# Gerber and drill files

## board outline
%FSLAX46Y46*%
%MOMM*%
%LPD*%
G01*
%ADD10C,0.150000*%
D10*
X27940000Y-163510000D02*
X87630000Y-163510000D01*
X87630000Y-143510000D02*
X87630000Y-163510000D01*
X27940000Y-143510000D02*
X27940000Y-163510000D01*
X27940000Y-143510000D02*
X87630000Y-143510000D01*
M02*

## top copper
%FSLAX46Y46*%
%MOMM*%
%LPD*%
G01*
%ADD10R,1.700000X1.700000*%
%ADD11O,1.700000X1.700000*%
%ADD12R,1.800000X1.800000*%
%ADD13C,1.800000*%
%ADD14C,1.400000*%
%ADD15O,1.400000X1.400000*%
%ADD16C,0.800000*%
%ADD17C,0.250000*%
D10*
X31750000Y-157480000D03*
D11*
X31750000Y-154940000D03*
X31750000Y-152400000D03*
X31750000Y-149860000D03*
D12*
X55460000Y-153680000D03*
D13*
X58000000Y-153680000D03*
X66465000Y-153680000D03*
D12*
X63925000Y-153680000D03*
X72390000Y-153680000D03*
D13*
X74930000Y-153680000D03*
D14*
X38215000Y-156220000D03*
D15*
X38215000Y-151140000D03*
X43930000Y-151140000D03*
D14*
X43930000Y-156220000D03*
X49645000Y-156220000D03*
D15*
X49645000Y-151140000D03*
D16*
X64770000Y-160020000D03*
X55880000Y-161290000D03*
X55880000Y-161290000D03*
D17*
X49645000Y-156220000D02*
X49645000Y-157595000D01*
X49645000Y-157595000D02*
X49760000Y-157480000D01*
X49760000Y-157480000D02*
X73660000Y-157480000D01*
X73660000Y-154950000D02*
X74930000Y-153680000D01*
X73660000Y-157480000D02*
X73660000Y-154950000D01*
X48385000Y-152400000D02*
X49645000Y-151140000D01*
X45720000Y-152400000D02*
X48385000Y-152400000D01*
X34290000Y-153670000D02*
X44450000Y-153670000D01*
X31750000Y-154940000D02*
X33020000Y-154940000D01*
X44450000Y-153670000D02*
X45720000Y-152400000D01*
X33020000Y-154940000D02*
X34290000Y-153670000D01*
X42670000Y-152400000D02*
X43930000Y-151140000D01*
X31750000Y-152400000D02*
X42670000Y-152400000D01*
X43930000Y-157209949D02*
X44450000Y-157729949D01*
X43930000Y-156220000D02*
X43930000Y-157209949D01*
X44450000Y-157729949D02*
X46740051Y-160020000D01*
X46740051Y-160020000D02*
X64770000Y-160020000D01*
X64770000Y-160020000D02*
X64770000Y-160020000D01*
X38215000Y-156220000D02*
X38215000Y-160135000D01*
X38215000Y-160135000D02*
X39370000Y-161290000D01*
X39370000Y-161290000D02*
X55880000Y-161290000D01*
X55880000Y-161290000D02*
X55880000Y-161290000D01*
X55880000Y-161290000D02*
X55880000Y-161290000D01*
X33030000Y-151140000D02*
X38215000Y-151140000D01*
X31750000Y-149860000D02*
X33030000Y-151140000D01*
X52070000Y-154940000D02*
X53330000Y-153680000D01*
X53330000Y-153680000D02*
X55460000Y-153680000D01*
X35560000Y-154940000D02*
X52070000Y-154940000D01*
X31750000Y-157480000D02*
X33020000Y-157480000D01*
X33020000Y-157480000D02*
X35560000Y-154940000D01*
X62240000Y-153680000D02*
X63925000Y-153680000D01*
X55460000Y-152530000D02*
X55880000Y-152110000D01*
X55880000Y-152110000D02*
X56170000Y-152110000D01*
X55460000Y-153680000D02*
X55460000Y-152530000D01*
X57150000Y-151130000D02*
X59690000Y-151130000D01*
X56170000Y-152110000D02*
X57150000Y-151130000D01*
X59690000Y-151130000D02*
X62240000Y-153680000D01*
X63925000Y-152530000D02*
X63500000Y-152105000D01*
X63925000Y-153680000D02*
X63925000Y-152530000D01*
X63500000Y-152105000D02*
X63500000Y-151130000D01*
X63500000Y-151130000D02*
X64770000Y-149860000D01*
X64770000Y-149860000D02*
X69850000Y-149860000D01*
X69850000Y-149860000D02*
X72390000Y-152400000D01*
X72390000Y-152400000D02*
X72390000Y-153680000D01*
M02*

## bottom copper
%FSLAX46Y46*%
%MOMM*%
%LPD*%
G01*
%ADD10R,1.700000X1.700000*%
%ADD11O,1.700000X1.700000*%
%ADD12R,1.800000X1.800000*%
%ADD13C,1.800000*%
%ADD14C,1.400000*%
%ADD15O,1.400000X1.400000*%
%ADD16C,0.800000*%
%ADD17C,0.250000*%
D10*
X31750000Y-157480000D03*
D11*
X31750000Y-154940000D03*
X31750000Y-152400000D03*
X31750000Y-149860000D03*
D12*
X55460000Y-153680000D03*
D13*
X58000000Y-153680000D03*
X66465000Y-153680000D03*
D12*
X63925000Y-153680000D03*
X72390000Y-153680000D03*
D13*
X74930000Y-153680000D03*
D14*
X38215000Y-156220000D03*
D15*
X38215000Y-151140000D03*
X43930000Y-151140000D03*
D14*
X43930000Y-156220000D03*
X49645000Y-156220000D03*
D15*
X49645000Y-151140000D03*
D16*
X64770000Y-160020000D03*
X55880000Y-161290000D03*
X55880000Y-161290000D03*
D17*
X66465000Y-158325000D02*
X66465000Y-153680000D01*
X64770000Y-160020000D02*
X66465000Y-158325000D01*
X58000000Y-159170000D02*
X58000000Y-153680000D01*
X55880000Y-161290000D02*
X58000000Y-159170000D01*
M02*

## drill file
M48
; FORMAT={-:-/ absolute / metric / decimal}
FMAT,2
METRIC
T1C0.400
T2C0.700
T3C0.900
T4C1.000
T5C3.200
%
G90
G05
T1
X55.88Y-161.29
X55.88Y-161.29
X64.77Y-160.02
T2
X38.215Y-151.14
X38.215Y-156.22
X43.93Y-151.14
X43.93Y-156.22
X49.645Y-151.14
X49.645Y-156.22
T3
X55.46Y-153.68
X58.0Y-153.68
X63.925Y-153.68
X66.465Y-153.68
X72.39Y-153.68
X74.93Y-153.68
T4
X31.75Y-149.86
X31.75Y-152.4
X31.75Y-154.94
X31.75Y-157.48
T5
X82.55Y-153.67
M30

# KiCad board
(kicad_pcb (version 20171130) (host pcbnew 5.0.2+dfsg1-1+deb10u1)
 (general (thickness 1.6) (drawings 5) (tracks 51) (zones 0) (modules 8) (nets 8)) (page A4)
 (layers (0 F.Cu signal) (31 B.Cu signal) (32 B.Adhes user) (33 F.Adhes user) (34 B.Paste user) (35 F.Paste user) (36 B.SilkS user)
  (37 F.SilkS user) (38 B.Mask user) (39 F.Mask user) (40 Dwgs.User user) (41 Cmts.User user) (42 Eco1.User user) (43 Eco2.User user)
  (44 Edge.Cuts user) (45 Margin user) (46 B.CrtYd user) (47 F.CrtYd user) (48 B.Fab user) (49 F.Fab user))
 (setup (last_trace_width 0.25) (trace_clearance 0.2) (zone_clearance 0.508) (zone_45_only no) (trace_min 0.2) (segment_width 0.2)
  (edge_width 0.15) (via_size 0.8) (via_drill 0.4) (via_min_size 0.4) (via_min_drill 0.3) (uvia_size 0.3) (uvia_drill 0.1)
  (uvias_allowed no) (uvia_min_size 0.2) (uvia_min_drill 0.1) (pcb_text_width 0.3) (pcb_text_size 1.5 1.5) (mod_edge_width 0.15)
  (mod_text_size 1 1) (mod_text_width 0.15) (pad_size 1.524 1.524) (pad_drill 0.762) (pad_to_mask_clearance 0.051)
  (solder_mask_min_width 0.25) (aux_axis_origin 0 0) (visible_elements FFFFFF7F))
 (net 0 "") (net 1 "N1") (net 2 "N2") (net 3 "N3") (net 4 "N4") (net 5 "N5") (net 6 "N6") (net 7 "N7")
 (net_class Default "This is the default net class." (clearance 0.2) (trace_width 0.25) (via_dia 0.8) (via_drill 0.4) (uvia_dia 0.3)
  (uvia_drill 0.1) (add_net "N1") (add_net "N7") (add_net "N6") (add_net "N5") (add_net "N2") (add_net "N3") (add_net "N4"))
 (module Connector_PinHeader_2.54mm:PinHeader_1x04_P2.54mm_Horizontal (layer F.Cu) (at 31.75 157.48 180)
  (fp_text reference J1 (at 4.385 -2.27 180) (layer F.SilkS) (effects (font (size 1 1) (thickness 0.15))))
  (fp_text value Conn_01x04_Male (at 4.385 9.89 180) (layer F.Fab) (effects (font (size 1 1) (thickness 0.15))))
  (pad 1 thru_hole rect (at 0 0 180) (size 1.7 1.7) (drill 1) (layers *.Cu *.Mask) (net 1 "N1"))
  (pad 2 thru_hole oval (at 0 2.54 180) (size 1.7 1.7) (drill 1) (layers *.Cu *.Mask) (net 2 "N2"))
  (pad 3 thru_hole oval (at 0 5.08 180) (size 1.7 1.7) (drill 1) (layers *.Cu *.Mask) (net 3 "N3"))
  (pad 4 thru_hole oval (at 0 7.62 180) (size 1.7 1.7) (drill 1) (layers *.Cu *.Mask) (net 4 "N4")))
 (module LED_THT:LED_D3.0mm (layer F.Cu) (at 55.46 153.68)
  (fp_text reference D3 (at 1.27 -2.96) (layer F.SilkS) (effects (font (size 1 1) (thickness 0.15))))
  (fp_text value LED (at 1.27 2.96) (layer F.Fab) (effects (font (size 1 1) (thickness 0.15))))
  (pad 1 thru_hole rect (at 0 0) (size 1.8 1.8) (drill 0.9) (layers *.Cu *.Mask) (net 1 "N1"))
  (pad 2 thru_hole circle (at 2.54 0) (size 1.8 1.8) (drill 0.9) (layers *.Cu *.Mask) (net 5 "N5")))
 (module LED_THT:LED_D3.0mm (layer F.Cu) (at 63.925 153.68)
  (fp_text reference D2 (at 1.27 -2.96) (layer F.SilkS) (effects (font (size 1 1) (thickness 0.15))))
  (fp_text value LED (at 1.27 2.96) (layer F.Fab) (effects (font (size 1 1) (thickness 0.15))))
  (pad 2 thru_hole circle (at 2.54 0) (size 1.8 1.8) (drill 0.9) (layers *.Cu *.Mask) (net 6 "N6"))
  (pad 1 thru_hole rect (at 0 0) (size 1.8 1.8) (drill 0.9) (layers *.Cu *.Mask) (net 1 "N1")))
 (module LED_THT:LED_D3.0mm (layer F.Cu) (at 72.39 153.68)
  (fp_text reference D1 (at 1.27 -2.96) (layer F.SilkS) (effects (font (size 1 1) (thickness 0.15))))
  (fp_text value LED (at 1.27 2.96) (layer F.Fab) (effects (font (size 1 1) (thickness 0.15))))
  (pad 1 thru_hole rect (at 0 0) (size 1.8 1.8) (drill 0.9) (layers *.Cu *.Mask) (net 1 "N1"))
  (pad 2 thru_hole circle (at 2.54 0) (size 1.8 1.8) (drill 0.9) (layers *.Cu *.Mask) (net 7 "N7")))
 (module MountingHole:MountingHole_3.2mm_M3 (layer F.Cu) (at 82.55 153.67)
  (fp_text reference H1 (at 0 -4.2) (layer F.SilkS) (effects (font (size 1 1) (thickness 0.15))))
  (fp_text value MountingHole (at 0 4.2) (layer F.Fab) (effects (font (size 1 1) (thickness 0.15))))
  (pad 1 np_thru_hole circle (at 0 0) (size 3.2 3.2) (drill 3.2) (layers *.Cu *.Mask)))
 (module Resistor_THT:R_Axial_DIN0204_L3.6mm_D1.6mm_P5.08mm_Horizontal (layer F.Cu) (at 38.215 156.22 90)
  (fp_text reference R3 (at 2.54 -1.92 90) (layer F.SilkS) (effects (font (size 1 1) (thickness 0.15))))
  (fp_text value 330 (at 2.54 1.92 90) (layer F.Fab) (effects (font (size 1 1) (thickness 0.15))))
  (pad 1 thru_hole circle (at 0 0 90) (size 1.4 1.4) (drill 0.7) (layers *.Cu *.Mask) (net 5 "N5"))
  (pad 2 thru_hole oval (at 5.08 0 90) (size 1.4 1.4) (drill 0.7) (layers *.Cu *.Mask) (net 4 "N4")))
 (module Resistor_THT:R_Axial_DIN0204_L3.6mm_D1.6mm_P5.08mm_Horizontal (layer F.Cu) (at 43.93 156.22 90)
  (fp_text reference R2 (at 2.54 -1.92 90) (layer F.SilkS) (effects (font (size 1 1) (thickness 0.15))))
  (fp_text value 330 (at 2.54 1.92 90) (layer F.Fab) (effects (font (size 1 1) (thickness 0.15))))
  (pad 2 thru_hole oval (at 5.08 0 90) (size 1.4 1.4) (drill 0.7) (layers *.Cu *.Mask) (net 3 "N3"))
  (pad 1 thru_hole circle (at 0 0 90) (size 1.4 1.4) (drill 0.7) (layers *.Cu *.Mask) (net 6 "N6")))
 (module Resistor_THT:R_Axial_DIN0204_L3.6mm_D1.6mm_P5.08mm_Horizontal (layer F.Cu) (at 49.645 156.22 90)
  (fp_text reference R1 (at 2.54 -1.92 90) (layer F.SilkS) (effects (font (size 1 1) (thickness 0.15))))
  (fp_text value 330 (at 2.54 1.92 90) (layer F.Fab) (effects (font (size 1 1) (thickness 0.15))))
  (pad 1 thru_hole circle (at 0 0 90) (size 1.4 1.4) (drill 0.7) (layers *.Cu *.Mask) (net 7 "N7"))
  (pad 2 thru_hole oval (at 5.08 0 90) (size 1.4 1.4) (drill 0.7) (layers *.Cu *.Mask) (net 2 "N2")))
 (gr_line (start 27.94 163.51) (end 87.63 163.51) (layer Edge.Cuts) (width 0.15))
 (gr_line (start 87.63 143.51) (end 87.63 163.51) (layer Edge.Cuts) (width 0.15))
 (gr_line (start 27.94 143.51) (end 27.94 163.51) (layer Edge.Cuts) (width 0.15))
 (gr_line (start 27.94 143.51) (end 87.63 143.51) (layer Edge.Cuts) (width 0.15))
 (segment (start 49.645 156.22) (end 49.645 157.595) (width 0.25) (layer F.Cu) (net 7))
 (segment (start 49.645 157.595) (end 49.76 157.48) (width 0.25) (layer F.Cu) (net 7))
 (segment (start 49.76 157.48) (end 73.66 157.48) (width 0.25) (layer F.Cu) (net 7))
 (segment (start 73.66 154.95) (end 74.93 153.68) (width 0.25) (layer F.Cu) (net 7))
 (segment (start 73.66 157.48) (end 73.66 154.95) (width 0.25) (layer F.Cu) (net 7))
 (segment (start 48.385 152.4) (end 49.645 151.14) (width 0.25) (layer F.Cu) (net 2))
 (segment (start 45.72 152.4) (end 48.385 152.4) (width 0.25) (layer F.Cu) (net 2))
 (segment (start 34.29 153.67) (end 44.45 153.67) (width 0.25) (layer F.Cu) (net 2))
 (segment (start 31.75 154.94) (end 33.02 154.94) (width 0.25) (layer F.Cu) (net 2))
 (segment (start 44.45 153.67) (end 45.72 152.4) (width 0.25) (layer F.Cu) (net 2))
 (segment (start 33.02 154.94) (end 34.29 153.67) (width 0.25) (layer F.Cu) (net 2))
 (segment (start 42.67 152.4) (end 43.93 151.14) (width 0.25) (layer F.Cu) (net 3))
 (segment (start 31.75 152.4) (end 42.67 152.4) (width 0.25) (layer F.Cu) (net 3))
 (segment (start 43.93 157.209949) (end 44.45 157.729949) (width 0.25) (layer F.Cu) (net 6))
 (segment (start 43.93 156.22) (end 43.93 157.209949) (width 0.25) (layer F.Cu) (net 6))
 (segment (start 44.45 157.729949) (end 46.740051 160.02) (width 0.25) (layer F.Cu) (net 6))
 (segment (start 46.740051 160.02) (end 64.77 160.02) (width 0.25) (layer F.Cu) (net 6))
 (segment (start 64.77 160.02) (end 64.77 160.02) (width 0.25) (layer F.Cu) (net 6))
 (via (at 64.77 160.02) (size 0.8) (drill 0.4) (layers F.Cu B.Cu) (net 6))
 (segment (start 66.465 158.325) (end 66.465 153.68) (width 0.25) (layer B.Cu) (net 6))
 (segment (start 64.77 160.02) (end 66.465 158.325) (width 0.25) (layer B.Cu) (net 6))
 (segment (start 38.215 156.22) (end 38.215 160.135) (width 0.25) (layer F.Cu) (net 5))
 (segment (start 38.215 160.135) (end 39.37 161.29) (width 0.25) (layer F.Cu) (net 5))
 (segment (start 39.37 161.29) (end 55.88 161.29) (width 0.25) (layer F.Cu) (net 5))
 (segment (start 55.88 161.29) (end 55.88 161.29) (width 0.25) (layer F.Cu) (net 5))
 (via (at 55.88 161.29) (size 0.8) (drill 0.4) (layers F.Cu B.Cu) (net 5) (status 1000000))
 (segment (start 55.88 161.29) (end 55.88 161.29) (width 0.25) (layer F.Cu) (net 5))
 (via (at 55.88 161.29) (size 0.8) (drill 0.4) (layers F.Cu B.Cu) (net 5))
 (segment (start 58 159.17) (end 58 153.68) (width 0.25) (layer B.Cu) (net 5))
 (segment (start 55.88 161.29) (end 58 159.17) (width 0.25) (layer B.Cu) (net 5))
 (segment (start 33.03 151.14) (end 38.215 151.14) (width 0.25) (layer F.Cu) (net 4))
 (segment (start 31.75 149.86) (end 33.03 151.14) (width 0.25) (layer F.Cu) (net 4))
 (segment (start 52.07 154.94) (end 53.33 153.68) (width 0.25) (layer F.Cu) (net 1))
 (segment (start 53.33 153.68) (end 55.46 153.68) (width 0.25) (layer F.Cu) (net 1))
 (segment (start 35.56 154.94) (end 52.07 154.94) (width 0.25) (layer F.Cu) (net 1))
 (segment (start 31.75 157.48) (end 33.02 157.48) (width 0.25) (layer F.Cu) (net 1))
 (segment (start 33.02 157.48) (end 35.56 154.94) (width 0.25) (layer F.Cu) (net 1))
 (segment (start 62.24 153.68) (end 63.925 153.68) (width 0.25) (layer F.Cu) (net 1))
 (segment (start 55.46 152.53) (end 55.88 152.11) (width 0.25) (layer F.Cu) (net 1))
 (segment (start 55.88 152.11) (end 56.17 152.11) (width 0.25) (layer F.Cu) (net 1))
 (segment (start 55.46 153.68) (end 55.46 152.53) (width 0.25) (layer F.Cu) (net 1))
 (segment (start 57.15 151.13) (end 59.69 151.13) (width 0.25) (layer F.Cu) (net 1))
 (segment (start 56.17 152.11) (end 57.15 151.13) (width 0.25) (layer F.Cu) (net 1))
 (segment (start 59.69 151.13) (end 62.24 153.68) (width 0.25) (layer F.Cu) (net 1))
 (segment (start 63.925 152.53) (end 63.5 152.105) (width 0.25) (layer F.Cu) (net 1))
 (segment (start 63.925 153.68) (end 63.925 152.53) (width 0.25) (layer F.Cu) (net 1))
 (segment (start 63.5 152.105) (end 63.5 151.13) (width 0.25) (layer F.Cu) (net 1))
 (segment (start 63.5 151.13) (end 64.77 149.86) (width 0.25) (layer F.Cu) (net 1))
 (segment (start 64.77 149.86) (end 69.85 149.86) (width 0.25) (layer F.Cu) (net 1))
 (segment (start 69.85 149.86) (end 72.39 152.4) (width 0.25) (layer F.Cu) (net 1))
 (segment (start 72.39 152.4) (end 72.39 153.68) (width 0.25) (layer F.Cu) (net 1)))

